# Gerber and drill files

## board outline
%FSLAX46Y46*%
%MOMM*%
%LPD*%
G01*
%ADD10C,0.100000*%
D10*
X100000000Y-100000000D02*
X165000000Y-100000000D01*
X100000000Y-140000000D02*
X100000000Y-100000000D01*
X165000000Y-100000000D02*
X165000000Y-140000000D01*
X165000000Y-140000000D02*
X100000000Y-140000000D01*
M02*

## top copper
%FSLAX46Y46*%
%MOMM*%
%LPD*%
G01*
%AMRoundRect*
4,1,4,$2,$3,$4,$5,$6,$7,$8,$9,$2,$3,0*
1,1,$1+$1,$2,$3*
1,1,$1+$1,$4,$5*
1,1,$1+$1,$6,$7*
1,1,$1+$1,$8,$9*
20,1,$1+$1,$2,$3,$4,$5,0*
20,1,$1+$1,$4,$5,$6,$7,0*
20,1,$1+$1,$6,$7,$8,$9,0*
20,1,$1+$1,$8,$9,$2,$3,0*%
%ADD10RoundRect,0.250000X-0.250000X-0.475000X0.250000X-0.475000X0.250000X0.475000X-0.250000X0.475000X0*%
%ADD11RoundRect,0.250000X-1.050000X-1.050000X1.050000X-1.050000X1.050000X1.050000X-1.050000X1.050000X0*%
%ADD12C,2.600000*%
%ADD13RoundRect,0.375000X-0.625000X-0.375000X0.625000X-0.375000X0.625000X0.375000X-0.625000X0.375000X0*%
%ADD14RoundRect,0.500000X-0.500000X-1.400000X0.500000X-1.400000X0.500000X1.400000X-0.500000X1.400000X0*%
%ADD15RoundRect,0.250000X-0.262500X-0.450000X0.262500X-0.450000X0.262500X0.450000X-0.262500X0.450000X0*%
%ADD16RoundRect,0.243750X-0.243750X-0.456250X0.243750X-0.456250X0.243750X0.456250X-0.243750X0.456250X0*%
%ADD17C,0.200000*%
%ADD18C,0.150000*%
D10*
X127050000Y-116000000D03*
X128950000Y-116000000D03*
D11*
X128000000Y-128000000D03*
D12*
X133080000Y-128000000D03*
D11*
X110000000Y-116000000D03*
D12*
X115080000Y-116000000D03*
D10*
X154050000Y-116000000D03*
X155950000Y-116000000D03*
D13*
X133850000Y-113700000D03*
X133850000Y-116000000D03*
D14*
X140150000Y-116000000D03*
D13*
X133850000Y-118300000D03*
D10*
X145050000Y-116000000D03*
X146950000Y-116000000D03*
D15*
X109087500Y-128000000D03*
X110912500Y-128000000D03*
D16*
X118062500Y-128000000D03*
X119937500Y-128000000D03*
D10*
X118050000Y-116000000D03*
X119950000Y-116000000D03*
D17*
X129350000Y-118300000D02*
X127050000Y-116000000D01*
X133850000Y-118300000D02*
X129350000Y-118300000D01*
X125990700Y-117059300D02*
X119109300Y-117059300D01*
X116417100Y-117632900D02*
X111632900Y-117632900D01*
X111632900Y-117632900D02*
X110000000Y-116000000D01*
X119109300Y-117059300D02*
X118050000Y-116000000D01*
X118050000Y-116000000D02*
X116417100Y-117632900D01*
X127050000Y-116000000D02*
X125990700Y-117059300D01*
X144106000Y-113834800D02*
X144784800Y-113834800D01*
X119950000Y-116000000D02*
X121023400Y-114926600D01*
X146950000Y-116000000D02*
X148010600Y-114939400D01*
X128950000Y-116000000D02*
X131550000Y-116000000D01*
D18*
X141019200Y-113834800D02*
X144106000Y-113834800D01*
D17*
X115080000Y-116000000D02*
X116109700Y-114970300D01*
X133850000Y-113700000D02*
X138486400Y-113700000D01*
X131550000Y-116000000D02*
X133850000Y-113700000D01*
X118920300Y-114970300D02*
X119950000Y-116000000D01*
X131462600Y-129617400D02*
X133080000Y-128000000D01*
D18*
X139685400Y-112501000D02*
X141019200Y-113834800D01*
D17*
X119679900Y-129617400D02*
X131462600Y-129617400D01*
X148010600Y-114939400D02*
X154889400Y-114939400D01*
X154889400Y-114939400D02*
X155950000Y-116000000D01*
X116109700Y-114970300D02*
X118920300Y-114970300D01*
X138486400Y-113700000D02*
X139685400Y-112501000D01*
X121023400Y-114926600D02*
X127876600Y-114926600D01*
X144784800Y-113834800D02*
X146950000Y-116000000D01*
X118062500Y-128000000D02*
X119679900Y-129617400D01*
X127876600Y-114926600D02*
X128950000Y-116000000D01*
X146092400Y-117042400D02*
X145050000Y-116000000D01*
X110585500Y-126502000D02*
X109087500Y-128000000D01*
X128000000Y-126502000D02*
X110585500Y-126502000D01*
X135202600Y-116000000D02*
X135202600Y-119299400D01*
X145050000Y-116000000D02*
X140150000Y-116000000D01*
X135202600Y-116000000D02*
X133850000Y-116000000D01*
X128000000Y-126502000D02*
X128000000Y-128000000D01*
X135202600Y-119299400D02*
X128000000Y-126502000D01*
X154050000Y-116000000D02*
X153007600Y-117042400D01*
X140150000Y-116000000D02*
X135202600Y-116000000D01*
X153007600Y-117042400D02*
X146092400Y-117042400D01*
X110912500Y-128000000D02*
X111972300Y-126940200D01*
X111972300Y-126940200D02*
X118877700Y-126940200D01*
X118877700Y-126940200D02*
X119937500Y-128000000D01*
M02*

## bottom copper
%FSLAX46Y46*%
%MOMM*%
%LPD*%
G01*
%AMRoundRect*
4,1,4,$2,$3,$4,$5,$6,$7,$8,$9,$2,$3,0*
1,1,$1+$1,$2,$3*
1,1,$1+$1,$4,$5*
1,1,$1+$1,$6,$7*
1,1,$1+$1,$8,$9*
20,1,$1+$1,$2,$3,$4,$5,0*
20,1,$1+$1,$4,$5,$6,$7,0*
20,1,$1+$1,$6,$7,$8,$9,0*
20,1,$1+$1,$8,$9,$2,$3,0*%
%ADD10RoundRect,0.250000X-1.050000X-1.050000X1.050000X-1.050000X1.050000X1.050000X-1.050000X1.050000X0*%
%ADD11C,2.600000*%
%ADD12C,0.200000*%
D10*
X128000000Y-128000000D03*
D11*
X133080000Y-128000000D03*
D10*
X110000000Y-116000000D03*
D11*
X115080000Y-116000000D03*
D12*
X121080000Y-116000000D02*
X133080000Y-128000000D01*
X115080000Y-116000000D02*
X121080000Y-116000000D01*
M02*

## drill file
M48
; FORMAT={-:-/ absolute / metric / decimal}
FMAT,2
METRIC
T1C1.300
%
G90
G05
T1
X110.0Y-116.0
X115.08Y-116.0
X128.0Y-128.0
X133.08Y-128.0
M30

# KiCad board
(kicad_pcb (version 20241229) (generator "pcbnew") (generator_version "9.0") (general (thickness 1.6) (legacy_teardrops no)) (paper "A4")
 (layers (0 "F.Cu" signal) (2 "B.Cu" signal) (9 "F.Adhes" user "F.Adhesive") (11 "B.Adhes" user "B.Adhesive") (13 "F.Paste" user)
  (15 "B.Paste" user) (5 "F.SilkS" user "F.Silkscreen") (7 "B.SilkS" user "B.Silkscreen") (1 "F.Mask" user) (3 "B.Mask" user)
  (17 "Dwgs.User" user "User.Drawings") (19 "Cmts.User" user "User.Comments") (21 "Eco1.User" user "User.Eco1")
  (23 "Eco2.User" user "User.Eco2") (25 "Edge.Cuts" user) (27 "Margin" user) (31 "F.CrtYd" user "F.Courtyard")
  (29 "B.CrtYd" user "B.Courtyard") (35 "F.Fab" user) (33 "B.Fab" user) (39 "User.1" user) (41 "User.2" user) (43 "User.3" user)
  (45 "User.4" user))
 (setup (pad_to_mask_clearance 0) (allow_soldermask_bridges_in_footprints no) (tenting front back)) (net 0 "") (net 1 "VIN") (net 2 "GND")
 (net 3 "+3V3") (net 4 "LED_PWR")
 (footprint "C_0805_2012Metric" (layer "F.Cu") (at 128 116)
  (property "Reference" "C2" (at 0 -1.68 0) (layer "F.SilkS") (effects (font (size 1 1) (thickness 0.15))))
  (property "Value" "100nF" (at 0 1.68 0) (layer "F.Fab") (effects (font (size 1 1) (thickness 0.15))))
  (pad "1" smd roundrect (at -0.95 0) (size 1 1.45) (layers "F.Cu" "F.Mask" "F.Paste") (roundrect_rratio 0.25) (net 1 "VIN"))
  (pad "2" smd roundrect (at 0.95 0) (size 1 1.45) (layers "F.Cu" "F.Mask" "F.Paste") (roundrect_rratio 0.25) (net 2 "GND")))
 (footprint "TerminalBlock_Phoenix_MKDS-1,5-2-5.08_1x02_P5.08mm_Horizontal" (layer "F.Cu") (at 128 128)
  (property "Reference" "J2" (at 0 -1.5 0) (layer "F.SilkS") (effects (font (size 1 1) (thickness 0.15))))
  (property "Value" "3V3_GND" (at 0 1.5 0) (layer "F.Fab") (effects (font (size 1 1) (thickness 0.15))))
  (pad "1" thru_hole roundrect (at 0 0) (size 2.6 2.6) (drill 1.3) (layers "*.Cu" "*.Mask") (remove_unused_layers no)
   (roundrect_rratio 0.096154) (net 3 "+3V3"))
  (pad "2" thru_hole circle (at 5.08 0) (size 2.6 2.6) (drill 1.3) (layers "*.Cu" "*.Mask") (remove_unused_layers no) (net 2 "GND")))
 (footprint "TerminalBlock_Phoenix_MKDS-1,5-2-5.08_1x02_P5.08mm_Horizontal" (layer "F.Cu") (at 110 116)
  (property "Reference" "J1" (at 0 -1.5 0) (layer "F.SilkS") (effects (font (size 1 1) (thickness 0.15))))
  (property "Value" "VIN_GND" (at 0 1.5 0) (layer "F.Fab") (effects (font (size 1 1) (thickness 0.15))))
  (pad "1" thru_hole roundrect (at 0 0) (size 2.6 2.6) (drill 1.3) (layers "*.Cu" "*.Mask") (remove_unused_layers no)
   (roundrect_rratio 0.096154) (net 1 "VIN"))
  (pad "2" thru_hole circle (at 5.08 0) (size 2.6 2.6) (drill 1.3) (layers "*.Cu" "*.Mask") (remove_unused_layers no) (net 2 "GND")))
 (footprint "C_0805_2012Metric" (layer "F.Cu") (at 155 116)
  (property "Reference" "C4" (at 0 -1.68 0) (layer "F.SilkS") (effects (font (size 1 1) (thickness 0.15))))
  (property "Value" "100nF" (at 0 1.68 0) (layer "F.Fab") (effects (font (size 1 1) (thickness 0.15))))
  (pad "1" smd roundrect (at -0.95 0) (size 1 1.45) (layers "F.Cu" "F.Mask" "F.Paste") (roundrect_rratio 0.25) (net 3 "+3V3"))
  (pad "2" smd roundrect (at 0.95 0) (size 1 1.45) (layers "F.Cu" "F.Mask" "F.Paste") (roundrect_rratio 0.25) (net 2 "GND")))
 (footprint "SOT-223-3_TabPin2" (layer "F.Cu") (at 137 116)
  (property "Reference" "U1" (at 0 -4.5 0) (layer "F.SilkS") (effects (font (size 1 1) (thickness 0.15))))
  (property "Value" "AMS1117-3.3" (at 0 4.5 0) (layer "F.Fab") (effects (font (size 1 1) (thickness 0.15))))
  (pad "1" smd roundrect (at -3.15 -2.3) (size 2 1.5) (layers "F.Cu" "F.Mask" "F.Paste") (roundrect_rratio 0.25) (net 2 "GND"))
  (pad "2" smd roundrect (at -3.15 0) (size 2 1.5) (layers "F.Cu" "F.Mask" "F.Paste") (roundrect_rratio 0.25) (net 3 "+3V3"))
  (pad "2" smd roundrect (at 3.15 0) (size 2 3.8) (layers "F.Cu" "F.Mask" "F.Paste") (roundrect_rratio 0.25) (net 3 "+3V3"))
  (pad "3" smd roundrect (at -3.15 2.3) (size 2 1.5) (layers "F.Cu" "F.Mask" "F.Paste") (roundrect_rratio 0.25) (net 1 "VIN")))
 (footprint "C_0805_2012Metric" (layer "F.Cu") (at 146 116)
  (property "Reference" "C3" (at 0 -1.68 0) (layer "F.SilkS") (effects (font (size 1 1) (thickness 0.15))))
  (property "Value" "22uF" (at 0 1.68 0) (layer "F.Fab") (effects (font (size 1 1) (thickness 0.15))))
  (pad "1" smd roundrect (at -0.95 0) (size 1 1.45) (layers "F.Cu" "F.Mask" "F.Paste") (roundrect_rratio 0.25) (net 3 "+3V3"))
  (pad "2" smd roundrect (at 0.95 0) (size 1 1.45) (layers "F.Cu" "F.Mask" "F.Paste") (roundrect_rratio 0.25) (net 2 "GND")))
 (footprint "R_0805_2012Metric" (layer "F.Cu") (at 110 128)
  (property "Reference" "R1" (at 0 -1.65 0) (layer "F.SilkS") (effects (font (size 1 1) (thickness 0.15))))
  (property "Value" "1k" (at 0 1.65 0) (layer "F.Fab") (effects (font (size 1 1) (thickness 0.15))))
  (pad "1" smd roundrect (at -0.9125 0) (size 1.025 1.4) (layers "F.Cu" "F.Mask" "F.Paste") (roundrect_rratio 0.243902) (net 3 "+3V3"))
  (pad "2" smd roundrect (at 0.9125 0) (size 1.025 1.4) (layers "F.Cu" "F.Mask" "F.Paste") (roundrect_rratio 0.243902) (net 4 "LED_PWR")))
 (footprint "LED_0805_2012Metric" (layer "F.Cu") (at 119 128)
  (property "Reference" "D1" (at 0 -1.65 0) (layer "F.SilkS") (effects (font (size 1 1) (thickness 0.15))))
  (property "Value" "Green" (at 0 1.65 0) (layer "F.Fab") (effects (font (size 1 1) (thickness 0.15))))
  (pad "1" smd roundrect (at -0.9375 0) (size 0.975 1.4) (layers "F.Cu" "F.Mask" "F.Paste") (roundrect_rratio 0.25) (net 2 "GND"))
  (pad "2" smd roundrect (at 0.9375 0) (size 0.975 1.4) (layers "F.Cu" "F.Mask" "F.Paste") (roundrect_rratio 0.25) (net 4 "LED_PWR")))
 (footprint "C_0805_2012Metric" (layer "F.Cu") (at 119 116)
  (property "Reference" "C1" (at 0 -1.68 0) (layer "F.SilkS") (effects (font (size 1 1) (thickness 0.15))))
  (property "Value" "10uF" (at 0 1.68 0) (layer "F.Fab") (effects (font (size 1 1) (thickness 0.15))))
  (pad "1" smd roundrect (at -0.95 0) (size 1 1.45) (layers "F.Cu" "F.Mask" "F.Paste") (roundrect_rratio 0.25) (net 1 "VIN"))
  (pad "2" smd roundrect (at 0.95 0) (size 1 1.45) (layers "F.Cu" "F.Mask" "F.Paste") (roundrect_rratio 0.25) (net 2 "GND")))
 (gr_line (start 100 100) (end 165 100) (stroke (width 0.1) (type default)) (layer "Edge.Cuts"))
 (gr_line (start 100 140) (end 100 100) (stroke (width 0.1) (type default)) (layer "Edge.Cuts"))
 (gr_line (start 165 100) (end 165 140) (stroke (width 0.1) (type default)) (layer "Edge.Cuts"))
 (gr_line (start 165 140) (end 100 140) (stroke (width 0.1) (type default)) (layer "Edge.Cuts"))
 (segment (start 129.35 118.3) (end 127.05 116) (width 0.2) (layer "F.Cu") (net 1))
 (segment (start 133.85 118.3) (end 129.35 118.3) (width 0.2) (layer "F.Cu") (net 1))
 (segment (start 125.9907 117.0593) (end 119.1093 117.0593) (width 0.2) (layer "F.Cu") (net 1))
 (segment (start 116.4171 117.6329) (end 111.6329 117.6329) (width 0.2) (layer "F.Cu") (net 1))
 (segment (start 111.6329 117.6329) (end 110 116) (width 0.2) (layer "F.Cu") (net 1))
 (segment (start 119.1093 117.0593) (end 118.05 116) (width 0.2) (layer "F.Cu") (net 1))
 (segment (start 118.05 116) (end 116.4171 117.6329) (width 0.2) (layer "F.Cu") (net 1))
 (segment (start 127.05 116) (end 125.9907 117.0593) (width 0.2) (layer "F.Cu") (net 1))
 (segment (start 144.106 113.8348) (end 144.7848 113.8348) (width 0.2) (layer "F.Cu") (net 2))
 (segment (start 119.95 116) (end 121.0234 114.9266) (width 0.2) (layer "F.Cu") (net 2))
 (segment (start 146.95 116) (end 148.0106 114.9394) (width 0.2) (layer "F.Cu") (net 2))
 (segment (start 128.95 116) (end 131.55 116) (width 0.2) (layer "F.Cu") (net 2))
 (segment (start 141.0192 113.8348) (end 144.106 113.8348) (width 0.15) (layer "F.Cu") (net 2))
 (segment (start 115.08 116) (end 116.1097 114.9703) (width 0.2) (layer "F.Cu") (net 2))
 (segment (start 133.85 113.7) (end 138.4864 113.7) (width 0.2) (layer "F.Cu") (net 2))
 (segment (start 131.55 116) (end 133.85 113.7) (width 0.2) (layer "F.Cu") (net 2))
 (segment (start 118.9203 114.9703) (end 119.95 116) (width 0.2) (layer "F.Cu") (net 2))
 (segment (start 131.4626 129.6174) (end 133.08 128) (width 0.2) (layer "F.Cu") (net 2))
 (segment (start 139.6854 112.501) (end 141.0192 113.8348) (width 0.15) (layer "F.Cu") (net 2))
 (segment (start 119.6799 129.6174) (end 131.4626 129.6174) (width 0.2) (layer "F.Cu") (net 2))
 (segment (start 148.0106 114.9394) (end 154.8894 114.9394) (width 0.2) (layer "F.Cu") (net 2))
 (segment (start 154.8894 114.9394) (end 155.95 116) (width 0.2) (layer "F.Cu") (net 2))
 (segment (start 116.1097 114.9703) (end 118.9203 114.9703) (width 0.2) (layer "F.Cu") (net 2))
 (segment (start 138.4864 113.7) (end 139.6854 112.501) (width 0.2) (layer "F.Cu") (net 2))
 (segment (start 121.0234 114.9266) (end 127.8766 114.9266) (width 0.2) (layer "F.Cu") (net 2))
 (segment (start 144.7848 113.8348) (end 146.95 116) (width 0.2) (layer "F.Cu") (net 2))
 (segment (start 118.0625 128) (end 119.6799 129.6174) (width 0.2) (layer "F.Cu") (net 2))
 (segment (start 127.8766 114.9266) (end 128.95 116) (width 0.2) (layer "F.Cu") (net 2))
 (segment (start 121.08 116) (end 133.08 128) (width 0.2) (layer "B.Cu") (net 2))
 (segment (start 115.08 116) (end 121.08 116) (width 0.2) (layer "B.Cu") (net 2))
 (segment (start 146.0924 117.0424) (end 145.05 116) (width 0.2) (layer "F.Cu") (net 3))
 (segment (start 110.5855 126.502) (end 109.0875 128) (width 0.2) (layer "F.Cu") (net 3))
 (segment (start 128 126.502) (end 110.5855 126.502) (width 0.2) (layer "F.Cu") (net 3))
 (segment (start 135.2026 116) (end 135.2026 119.2994) (width 0.2) (layer "F.Cu") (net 3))
 (segment (start 145.05 116) (end 140.15 116) (width 0.2) (layer "F.Cu") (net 3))
 (segment (start 135.2026 116) (end 133.85 116) (width 0.2) (layer "F.Cu") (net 3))
 (segment (start 128 126.502) (end 128 128) (width 0.2) (layer "F.Cu") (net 3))
 (segment (start 135.2026 119.2994) (end 128 126.502) (width 0.2) (layer "F.Cu") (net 3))
 (segment (start 154.05 116) (end 153.0076 117.0424) (width 0.2) (layer "F.Cu") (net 3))
 (segment (start 140.15 116) (end 135.2026 116) (width 0.2) (layer "F.Cu") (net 3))
 (segment (start 153.0076 117.0424) (end 146.0924 117.0424) (width 0.2) (layer "F.Cu") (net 3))
 (segment (start 110.9125 128) (end 111.9723 126.9402) (width 0.2) (layer "F.Cu") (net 4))
 (segment (start 111.9723 126.9402) (end 118.8777 126.9402) (width 0.2) (layer "F.Cu") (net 4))
 (segment (start 118.8777 126.9402) (end 119.9375 128) (width 0.2) (layer "F.Cu") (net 4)))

